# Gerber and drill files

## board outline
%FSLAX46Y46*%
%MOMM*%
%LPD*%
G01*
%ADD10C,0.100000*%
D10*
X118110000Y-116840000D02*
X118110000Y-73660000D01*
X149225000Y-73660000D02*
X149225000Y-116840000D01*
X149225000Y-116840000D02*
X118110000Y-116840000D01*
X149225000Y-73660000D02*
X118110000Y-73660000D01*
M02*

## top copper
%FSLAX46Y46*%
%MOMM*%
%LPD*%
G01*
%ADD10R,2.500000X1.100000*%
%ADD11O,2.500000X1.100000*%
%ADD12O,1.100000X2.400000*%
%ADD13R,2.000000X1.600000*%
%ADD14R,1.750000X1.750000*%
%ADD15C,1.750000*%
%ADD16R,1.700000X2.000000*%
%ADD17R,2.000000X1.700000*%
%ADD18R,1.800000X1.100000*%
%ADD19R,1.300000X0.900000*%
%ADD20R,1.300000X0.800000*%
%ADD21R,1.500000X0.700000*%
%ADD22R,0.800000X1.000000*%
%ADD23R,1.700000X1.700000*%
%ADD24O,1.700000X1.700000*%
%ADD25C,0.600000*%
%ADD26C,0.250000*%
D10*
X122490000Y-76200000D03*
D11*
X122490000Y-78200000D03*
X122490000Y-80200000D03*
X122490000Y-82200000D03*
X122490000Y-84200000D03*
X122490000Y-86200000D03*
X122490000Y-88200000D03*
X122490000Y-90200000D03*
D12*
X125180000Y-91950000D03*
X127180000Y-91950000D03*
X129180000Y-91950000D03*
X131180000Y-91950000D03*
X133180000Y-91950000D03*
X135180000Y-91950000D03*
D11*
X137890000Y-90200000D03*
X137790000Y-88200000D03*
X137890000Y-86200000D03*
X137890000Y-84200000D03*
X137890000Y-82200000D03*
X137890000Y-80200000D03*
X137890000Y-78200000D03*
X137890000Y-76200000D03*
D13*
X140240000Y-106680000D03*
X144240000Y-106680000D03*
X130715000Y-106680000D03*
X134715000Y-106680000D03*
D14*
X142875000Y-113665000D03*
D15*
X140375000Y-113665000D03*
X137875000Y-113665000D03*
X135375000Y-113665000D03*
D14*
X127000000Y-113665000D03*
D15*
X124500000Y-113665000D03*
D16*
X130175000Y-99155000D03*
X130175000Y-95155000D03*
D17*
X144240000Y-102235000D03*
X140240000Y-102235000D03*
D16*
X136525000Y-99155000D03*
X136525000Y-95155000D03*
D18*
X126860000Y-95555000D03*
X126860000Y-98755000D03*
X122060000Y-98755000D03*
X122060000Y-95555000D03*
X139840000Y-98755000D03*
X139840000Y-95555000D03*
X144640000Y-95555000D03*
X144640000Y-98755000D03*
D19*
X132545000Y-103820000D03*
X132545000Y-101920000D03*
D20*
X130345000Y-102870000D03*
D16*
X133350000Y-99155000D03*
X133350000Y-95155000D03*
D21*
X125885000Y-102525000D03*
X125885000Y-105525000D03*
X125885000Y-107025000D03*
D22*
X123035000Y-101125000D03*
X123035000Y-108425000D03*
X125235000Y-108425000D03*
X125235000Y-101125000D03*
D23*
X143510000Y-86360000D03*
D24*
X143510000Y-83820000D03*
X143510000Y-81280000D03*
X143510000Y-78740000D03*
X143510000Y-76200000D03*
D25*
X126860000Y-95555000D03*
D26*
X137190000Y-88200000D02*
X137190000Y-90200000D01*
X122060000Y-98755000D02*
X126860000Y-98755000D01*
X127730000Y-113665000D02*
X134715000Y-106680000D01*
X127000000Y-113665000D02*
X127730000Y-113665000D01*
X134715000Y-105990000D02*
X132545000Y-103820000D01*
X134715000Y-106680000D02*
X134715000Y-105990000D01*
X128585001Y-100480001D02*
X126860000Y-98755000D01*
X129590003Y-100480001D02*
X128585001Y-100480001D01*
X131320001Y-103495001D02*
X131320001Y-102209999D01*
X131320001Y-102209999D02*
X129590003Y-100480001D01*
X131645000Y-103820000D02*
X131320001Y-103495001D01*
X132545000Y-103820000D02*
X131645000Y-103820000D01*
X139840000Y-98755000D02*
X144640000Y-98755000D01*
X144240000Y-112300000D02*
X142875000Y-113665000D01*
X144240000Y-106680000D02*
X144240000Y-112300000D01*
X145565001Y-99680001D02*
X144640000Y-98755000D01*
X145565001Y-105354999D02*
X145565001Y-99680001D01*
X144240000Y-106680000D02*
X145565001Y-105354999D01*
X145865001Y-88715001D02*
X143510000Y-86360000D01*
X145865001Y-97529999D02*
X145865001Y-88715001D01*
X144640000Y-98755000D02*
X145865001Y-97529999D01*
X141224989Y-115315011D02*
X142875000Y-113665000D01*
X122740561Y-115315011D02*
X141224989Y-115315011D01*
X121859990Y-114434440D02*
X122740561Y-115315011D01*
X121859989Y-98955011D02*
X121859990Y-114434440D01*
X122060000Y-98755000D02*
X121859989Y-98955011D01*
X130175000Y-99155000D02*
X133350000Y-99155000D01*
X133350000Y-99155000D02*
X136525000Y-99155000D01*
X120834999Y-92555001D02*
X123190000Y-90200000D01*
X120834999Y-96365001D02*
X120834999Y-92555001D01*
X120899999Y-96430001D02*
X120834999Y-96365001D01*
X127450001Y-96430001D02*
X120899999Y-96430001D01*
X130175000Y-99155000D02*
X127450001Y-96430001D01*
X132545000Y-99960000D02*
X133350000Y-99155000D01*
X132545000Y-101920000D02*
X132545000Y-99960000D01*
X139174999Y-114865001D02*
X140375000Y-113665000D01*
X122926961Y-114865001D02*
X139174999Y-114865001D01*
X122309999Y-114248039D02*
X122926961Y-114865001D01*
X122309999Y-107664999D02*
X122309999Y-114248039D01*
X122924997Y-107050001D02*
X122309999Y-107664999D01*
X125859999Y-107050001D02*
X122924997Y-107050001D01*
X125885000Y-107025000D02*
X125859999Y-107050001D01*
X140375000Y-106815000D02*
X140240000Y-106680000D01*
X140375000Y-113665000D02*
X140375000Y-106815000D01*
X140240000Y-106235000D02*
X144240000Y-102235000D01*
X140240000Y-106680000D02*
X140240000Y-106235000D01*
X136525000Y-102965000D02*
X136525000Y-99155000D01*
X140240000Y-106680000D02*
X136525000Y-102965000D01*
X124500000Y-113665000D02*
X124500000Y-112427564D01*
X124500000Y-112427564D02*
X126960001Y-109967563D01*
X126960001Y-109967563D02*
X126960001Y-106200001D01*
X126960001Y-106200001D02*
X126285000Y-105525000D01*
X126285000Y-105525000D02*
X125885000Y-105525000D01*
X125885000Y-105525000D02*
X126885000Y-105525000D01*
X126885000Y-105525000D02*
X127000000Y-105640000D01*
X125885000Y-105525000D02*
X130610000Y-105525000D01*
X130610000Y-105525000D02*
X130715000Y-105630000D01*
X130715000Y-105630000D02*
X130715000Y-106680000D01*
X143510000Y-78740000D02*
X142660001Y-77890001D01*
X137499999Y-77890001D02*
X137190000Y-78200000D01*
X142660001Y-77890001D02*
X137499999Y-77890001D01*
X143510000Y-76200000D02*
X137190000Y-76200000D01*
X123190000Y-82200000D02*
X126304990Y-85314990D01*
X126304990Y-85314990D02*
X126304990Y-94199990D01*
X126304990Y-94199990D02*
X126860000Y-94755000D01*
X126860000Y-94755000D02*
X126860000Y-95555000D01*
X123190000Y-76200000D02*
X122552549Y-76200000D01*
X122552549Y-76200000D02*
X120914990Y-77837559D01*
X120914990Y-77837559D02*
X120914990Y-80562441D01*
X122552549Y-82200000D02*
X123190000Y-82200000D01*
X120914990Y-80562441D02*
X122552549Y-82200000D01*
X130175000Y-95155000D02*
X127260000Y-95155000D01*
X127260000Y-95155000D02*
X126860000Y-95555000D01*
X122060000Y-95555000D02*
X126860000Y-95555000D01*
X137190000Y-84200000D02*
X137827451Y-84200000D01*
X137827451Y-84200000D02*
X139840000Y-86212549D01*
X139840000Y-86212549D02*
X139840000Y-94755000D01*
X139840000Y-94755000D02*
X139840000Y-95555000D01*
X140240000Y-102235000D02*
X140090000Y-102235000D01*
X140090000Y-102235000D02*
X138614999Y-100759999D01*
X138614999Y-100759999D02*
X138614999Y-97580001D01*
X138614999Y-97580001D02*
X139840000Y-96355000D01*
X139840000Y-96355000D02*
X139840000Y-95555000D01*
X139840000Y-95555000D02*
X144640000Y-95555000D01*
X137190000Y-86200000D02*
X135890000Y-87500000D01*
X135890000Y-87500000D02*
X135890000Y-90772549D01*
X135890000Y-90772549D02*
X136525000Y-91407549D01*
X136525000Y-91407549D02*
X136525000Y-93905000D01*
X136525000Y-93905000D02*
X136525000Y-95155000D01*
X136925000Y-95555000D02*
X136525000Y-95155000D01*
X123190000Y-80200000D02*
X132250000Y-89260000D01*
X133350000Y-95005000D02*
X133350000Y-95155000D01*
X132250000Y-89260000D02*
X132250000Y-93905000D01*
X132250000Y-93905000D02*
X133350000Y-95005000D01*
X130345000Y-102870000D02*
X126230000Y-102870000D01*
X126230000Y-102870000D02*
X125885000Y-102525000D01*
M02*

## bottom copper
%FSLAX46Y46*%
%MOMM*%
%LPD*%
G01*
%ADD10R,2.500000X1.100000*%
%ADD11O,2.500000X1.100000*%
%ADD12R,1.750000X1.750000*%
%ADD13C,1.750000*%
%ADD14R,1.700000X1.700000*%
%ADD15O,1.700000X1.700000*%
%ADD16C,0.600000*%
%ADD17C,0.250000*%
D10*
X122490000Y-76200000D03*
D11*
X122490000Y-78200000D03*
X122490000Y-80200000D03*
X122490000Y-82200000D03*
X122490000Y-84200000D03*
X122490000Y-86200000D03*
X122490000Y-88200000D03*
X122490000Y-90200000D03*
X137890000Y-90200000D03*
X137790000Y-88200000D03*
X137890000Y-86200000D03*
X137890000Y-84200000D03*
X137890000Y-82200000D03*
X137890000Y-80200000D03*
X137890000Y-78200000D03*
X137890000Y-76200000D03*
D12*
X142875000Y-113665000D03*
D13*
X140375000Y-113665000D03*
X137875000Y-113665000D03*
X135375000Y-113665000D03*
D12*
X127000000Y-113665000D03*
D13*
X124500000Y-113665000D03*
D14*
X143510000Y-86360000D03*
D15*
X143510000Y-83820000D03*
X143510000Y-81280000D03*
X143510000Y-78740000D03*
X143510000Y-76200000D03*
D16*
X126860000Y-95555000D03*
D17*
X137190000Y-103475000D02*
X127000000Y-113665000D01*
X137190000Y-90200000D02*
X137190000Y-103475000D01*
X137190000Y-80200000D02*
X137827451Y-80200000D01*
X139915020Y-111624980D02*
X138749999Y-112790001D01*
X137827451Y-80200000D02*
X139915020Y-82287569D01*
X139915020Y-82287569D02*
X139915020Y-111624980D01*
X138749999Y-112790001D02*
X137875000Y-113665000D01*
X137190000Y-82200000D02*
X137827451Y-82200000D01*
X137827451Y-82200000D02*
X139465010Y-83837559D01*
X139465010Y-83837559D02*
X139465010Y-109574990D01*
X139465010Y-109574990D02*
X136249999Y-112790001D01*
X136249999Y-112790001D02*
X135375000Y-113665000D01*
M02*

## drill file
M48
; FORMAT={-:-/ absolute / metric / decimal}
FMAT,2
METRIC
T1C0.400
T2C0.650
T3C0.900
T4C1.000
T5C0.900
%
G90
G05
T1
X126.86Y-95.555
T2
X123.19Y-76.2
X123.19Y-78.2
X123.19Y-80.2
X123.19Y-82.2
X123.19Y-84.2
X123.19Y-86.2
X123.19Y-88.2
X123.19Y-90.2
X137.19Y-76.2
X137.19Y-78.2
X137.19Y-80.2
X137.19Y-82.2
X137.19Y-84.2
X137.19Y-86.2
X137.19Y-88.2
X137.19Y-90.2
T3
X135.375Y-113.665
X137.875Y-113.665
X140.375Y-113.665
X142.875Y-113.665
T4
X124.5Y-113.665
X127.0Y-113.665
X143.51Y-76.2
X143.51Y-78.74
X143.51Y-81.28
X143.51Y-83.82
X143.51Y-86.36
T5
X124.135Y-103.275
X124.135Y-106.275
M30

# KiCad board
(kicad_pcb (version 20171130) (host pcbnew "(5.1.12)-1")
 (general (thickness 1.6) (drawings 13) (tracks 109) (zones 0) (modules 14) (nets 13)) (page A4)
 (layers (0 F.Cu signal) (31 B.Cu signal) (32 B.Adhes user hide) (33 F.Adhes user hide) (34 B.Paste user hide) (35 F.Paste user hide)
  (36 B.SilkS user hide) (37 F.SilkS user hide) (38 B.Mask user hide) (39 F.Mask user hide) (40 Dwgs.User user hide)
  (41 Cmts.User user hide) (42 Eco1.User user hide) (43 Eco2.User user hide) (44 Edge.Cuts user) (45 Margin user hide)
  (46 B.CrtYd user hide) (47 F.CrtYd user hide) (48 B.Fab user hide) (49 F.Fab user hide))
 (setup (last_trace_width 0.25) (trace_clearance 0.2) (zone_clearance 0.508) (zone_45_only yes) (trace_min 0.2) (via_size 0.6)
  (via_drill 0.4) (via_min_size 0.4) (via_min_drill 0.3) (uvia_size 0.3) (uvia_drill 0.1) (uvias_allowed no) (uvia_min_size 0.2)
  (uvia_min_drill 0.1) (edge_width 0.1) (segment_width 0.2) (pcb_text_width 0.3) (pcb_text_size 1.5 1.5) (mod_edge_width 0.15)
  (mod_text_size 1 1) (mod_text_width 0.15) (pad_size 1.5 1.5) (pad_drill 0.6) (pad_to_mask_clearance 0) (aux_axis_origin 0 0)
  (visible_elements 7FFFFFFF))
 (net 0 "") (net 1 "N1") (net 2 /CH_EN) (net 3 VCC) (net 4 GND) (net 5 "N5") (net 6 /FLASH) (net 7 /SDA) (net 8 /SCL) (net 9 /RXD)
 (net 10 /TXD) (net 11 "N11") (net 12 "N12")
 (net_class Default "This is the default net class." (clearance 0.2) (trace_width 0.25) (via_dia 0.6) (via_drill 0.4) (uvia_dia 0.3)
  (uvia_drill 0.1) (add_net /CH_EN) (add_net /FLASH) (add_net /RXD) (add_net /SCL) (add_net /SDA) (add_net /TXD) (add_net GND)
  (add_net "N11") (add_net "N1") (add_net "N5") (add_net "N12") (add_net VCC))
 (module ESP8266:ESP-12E (layer F.Cu) (at 123.19 76.2)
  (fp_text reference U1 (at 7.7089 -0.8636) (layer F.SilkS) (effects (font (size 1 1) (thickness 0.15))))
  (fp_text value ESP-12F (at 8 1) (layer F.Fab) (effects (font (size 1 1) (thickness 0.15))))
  (pad 1 thru_hole rect (at 0 0) (size 2.5 1.1) (drill 0.65 (offset -0.7 0)) (layers *.Cu *.Mask F.SilkS) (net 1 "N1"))
  (pad 2 thru_hole oval (at 0 2) (size 2.5 1.1) (drill 0.65 (offset -0.7 0)) (layers *.Cu *.Mask F.SilkS))
  (pad 3 thru_hole oval (at 0 4) (size 2.5 1.1) (drill 0.65 (offset -0.7 0)) (layers *.Cu *.Mask F.SilkS) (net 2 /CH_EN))
  (pad 4 thru_hole oval (at 0 6) (size 2.5 1.1) (drill 0.65 (offset -0.7 0)) (layers *.Cu *.Mask F.SilkS) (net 1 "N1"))
  (pad 5 thru_hole oval (at 0 8) (size 2.5 1.1) (drill 0.65 (offset -0.7 0)) (layers *.Cu *.Mask F.SilkS))
  (pad 6 thru_hole oval (at 0 10) (size 2.5 1.1) (drill 0.65 (offset -0.7 0)) (layers *.Cu *.Mask F.SilkS))
  (pad 7 thru_hole oval (at 0 12) (size 2.5 1.1) (drill 0.65 (offset -0.7 0)) (layers *.Cu *.Mask F.SilkS))
  (pad 8 thru_hole oval (at 0 14) (size 2.5 1.1) (drill 0.65 (offset -0.7 0)) (layers *.Cu *.Mask F.SilkS) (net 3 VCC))
  (pad 9 smd oval (at 1.99 15.75 90) (size 2.4 1.1) (layers F.Cu F.Paste F.Mask))
  (pad 10 smd oval (at 3.99 15.75 90) (size 2.4 1.1) (layers F.Cu F.Paste F.Mask))
  (pad 11 smd oval (at 5.99 15.75 90) (size 2.4 1.1) (layers F.Cu F.Paste F.Mask))
  (pad 12 smd oval (at 7.99 15.75 90) (size 2.4 1.1) (layers F.Cu F.Paste F.Mask))
  (pad 13 smd oval (at 9.99 15.75 90) (size 2.4 1.1) (layers F.Cu F.Paste F.Mask))
  (pad 14 smd oval (at 11.99 15.75 90) (size 2.4 1.1) (layers F.Cu F.Paste F.Mask))
  (pad 15 thru_hole oval (at 14 14) (size 2.5 1.1) (drill 0.65 (offset 0.7 0)) (layers *.Cu *.Mask F.SilkS) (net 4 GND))
  (pad 16 thru_hole oval (at 14 12) (size 2.5 1.1) (drill 0.65 (offset 0.6 0)) (layers *.Cu *.Mask F.SilkS) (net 4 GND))
  (pad 17 thru_hole oval (at 14 10) (size 2.5 1.1) (drill 0.65 (offset 0.7 0)) (layers *.Cu *.Mask F.SilkS) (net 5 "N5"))
  (pad 18 thru_hole oval (at 14 8) (size 2.5 1.1) (drill 0.65 (offset 0.7 0)) (layers *.Cu *.Mask F.SilkS) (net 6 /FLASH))
  (pad 19 thru_hole oval (at 14 6) (size 2.5 1.1) (drill 0.65 (offset 0.7 0)) (layers *.Cu *.Mask F.SilkS) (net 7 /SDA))
  (pad 20 thru_hole oval (at 14 4) (size 2.5 1.1) (drill 0.65 (offset 0.7 0)) (layers *.Cu *.Mask F.SilkS) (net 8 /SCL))
  (pad 21 thru_hole oval (at 14 2) (size 2.5 1.1) (drill 0.65 (offset 0.7 0)) (layers *.Cu *.Mask F.SilkS) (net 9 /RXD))
  (pad 22 thru_hole oval (at 14 0) (size 2.5 1.1) (drill 0.65 (offset 0.7 0)) (layers *.Cu *.Mask F.SilkS) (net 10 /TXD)))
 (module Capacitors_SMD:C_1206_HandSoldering (layer F.Cu) (at 142.24 106.68)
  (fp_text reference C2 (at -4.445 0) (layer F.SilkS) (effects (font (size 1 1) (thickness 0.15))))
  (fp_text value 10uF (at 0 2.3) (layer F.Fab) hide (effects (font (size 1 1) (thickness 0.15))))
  (pad 1 smd rect (at -2 0) (size 2 1.6) (layers F.Cu F.Paste F.Mask) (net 3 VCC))
  (pad 2 smd rect (at 2 0) (size 2 1.6) (layers F.Cu F.Paste F.Mask) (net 4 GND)))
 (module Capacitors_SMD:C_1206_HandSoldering (layer F.Cu) (at 132.715 106.68)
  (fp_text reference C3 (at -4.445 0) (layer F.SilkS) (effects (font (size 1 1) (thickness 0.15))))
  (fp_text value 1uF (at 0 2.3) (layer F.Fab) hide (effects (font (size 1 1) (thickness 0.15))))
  (pad 1 smd rect (at -2 0) (size 2 1.6) (layers F.Cu F.Paste F.Mask) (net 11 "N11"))
  (pad 2 smd rect (at 2 0) (size 2 1.6) (layers F.Cu F.Paste F.Mask) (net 4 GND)))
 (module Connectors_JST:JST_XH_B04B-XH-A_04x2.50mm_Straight (layer F.Cu) (at 142.875 113.665 180)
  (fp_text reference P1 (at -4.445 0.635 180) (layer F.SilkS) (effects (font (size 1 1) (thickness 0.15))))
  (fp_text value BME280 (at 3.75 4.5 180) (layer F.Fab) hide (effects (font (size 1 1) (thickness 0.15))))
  (pad 1 thru_hole rect (at 0 0 180) (size 1.75 1.75) (drill 0.9) (layers *.Cu *.Mask) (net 4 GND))
  (pad 2 thru_hole circle (at 2.5 0 180) (size 1.75 1.75) (drill 0.9) (layers *.Cu *.Mask) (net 3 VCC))
  (pad 3 thru_hole circle (at 5 0 180) (size 1.75 1.75) (drill 0.9) (layers *.Cu *.Mask) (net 8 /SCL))
  (pad 4 thru_hole circle (at 7.5 0 180) (size 1.75 1.75) (drill 0.9) (layers *.Cu *.Mask) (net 7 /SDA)))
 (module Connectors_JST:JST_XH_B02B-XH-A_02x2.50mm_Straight (layer F.Cu) (at 127 113.665 180)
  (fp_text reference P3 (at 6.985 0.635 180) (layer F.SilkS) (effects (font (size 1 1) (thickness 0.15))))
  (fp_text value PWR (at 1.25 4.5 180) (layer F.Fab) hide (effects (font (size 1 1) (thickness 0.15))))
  (pad 1 thru_hole rect (at 0 0 180) (size 1.75 1.75) (drill 1) (layers *.Cu *.Mask) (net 4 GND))
  (pad 2 thru_hole circle (at 2.5 0 180) (size 1.75 1.75) (drill 1) (layers *.Cu *.Mask) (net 11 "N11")))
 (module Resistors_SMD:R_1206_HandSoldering (layer F.Cu) (at 130.175 97.155 90)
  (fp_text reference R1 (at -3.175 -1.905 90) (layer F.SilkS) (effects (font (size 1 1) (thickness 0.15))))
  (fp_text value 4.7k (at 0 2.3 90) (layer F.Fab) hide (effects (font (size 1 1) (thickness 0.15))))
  (pad 1 smd rect (at -2 0 90) (size 2 1.7) (layers F.Cu F.Paste F.Mask) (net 3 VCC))
  (pad 2 smd rect (at 2 0 90) (size 2 1.7) (layers F.Cu F.Paste F.Mask) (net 1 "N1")))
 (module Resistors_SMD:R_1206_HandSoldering (layer F.Cu) (at 142.24 102.235 180)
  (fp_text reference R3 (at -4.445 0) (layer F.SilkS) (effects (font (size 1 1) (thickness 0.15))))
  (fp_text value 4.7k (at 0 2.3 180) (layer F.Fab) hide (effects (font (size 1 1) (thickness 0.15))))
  (pad 1 smd rect (at -2 0 180) (size 2 1.7) (layers F.Cu F.Paste F.Mask) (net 3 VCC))
  (pad 2 smd rect (at 2 0 180) (size 2 1.7) (layers F.Cu F.Paste F.Mask) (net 6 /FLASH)))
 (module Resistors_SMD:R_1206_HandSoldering (layer F.Cu) (at 136.525 97.155 90)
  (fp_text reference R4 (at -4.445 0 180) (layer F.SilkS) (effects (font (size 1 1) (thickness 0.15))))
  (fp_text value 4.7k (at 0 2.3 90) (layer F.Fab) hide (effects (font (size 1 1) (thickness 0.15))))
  (pad 1 smd rect (at -2 0 90) (size 2 1.7) (layers F.Cu F.Paste F.Mask) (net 3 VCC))
  (pad 2 smd rect (at 2 0 90) (size 2 1.7) (layers F.Cu F.Paste F.Mask) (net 5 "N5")))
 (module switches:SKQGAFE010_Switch (layer F.Cu) (at 124.46 97.155 180)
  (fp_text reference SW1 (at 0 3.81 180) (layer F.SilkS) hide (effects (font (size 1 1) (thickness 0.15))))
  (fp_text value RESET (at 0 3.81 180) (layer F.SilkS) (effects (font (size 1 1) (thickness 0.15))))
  (pad 3 smd rect (at -2.4 1.6 180) (size 1.8 1.1) (layers F.Cu F.Paste F.Mask) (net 1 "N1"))
  (pad 1 smd rect (at -2.4 -1.6 180) (size 1.8 1.1) (layers F.Cu F.Paste F.Mask) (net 4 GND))
  (pad 2 smd rect (at 2.4 -1.6 180) (size 1.8 1.1) (layers F.Cu F.Paste F.Mask) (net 4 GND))
  (pad 4 smd rect (at 2.4 1.6 180) (size 1.8 1.1) (layers F.Cu F.Paste F.Mask) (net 1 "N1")))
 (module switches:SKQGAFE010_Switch (layer F.Cu) (at 142.24 97.155)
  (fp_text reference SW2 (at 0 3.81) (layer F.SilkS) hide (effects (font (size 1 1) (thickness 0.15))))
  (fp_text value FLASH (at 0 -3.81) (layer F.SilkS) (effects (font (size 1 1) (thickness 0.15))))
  (pad 3 smd rect (at -2.4 1.6) (size 1.8 1.1) (layers F.Cu F.Paste F.Mask) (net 4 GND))
  (pad 1 smd rect (at -2.4 -1.6) (size 1.8 1.1) (layers F.Cu F.Paste F.Mask) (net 6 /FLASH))
  (pad 2 smd rect (at 2.4 -1.6) (size 1.8 1.1) (layers F.Cu F.Paste F.Mask) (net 6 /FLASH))
  (pad 4 smd rect (at 2.4 1.6) (size 1.8 1.1) (layers F.Cu F.Paste F.Mask) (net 4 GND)))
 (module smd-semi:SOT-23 (layer F.Cu) (at 131.445 102.87 180)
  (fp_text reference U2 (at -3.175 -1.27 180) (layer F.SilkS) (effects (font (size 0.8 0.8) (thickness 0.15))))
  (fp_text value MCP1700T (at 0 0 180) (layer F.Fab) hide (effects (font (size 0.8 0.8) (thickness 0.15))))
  (pad 1 smd rect (at -1.1 -0.95 180) (size 1.3 0.9) (layers F.Cu F.Paste F.Mask) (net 4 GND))
  (pad 2 smd rect (at -1.1 0.95 180) (size 1.3 0.9) (layers F.Cu F.Paste F.Mask) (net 3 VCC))
  (pad 3 smd rect (at 1.1 0 180) (size 1.3 0.8) (layers F.Cu F.Paste F.Mask) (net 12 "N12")))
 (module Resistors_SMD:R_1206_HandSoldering (layer F.Cu) (at 133.35 97.155 90)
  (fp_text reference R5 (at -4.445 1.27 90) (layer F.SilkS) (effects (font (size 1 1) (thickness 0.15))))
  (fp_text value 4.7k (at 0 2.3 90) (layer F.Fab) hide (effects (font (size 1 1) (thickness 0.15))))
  (pad 1 smd rect (at -2 0 90) (size 2 1.7) (layers F.Cu F.Paste F.Mask) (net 3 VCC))
  (pad 2 smd rect (at 2 0 90) (size 2 1.7) (layers F.Cu F.Paste F.Mask) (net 2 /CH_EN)))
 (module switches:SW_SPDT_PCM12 (layer F.Cu) (at 124.46 104.775 270)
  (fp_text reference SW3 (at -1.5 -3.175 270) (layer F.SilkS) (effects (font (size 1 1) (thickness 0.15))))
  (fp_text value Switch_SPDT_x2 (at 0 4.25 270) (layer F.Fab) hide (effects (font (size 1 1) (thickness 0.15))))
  (pad "" np_thru_hole circle (at -1.5 0.325 270) (size 0.9 0.9) (drill 0.9) (layers *.Cu *.Mask))
  (pad "" np_thru_hole circle (at 1.5 0.325 270) (size 0.9 0.9) (drill 0.9) (layers *.Cu *.Mask))
  (pad 1 smd rect (at -2.25 -1.425 270) (size 0.7 1.5) (layers F.Cu F.Paste F.Mask) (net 12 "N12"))
  (pad 2 smd rect (at 0.75 -1.425 270) (size 0.7 1.5) (layers F.Cu F.Paste F.Mask) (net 11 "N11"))
  (pad 3 smd rect (at 2.25 -1.425 270) (size 0.7 1.5) (layers F.Cu F.Paste F.Mask) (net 3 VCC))
  (pad "" smd rect (at -3.65 1.425 270) (size 1 0.8) (layers F.Cu F.Paste F.Mask))
  (pad "" smd rect (at 3.65 1.425 270) (size 1 0.8) (layers F.Cu F.Paste F.Mask))
  (pad "" smd rect (at 3.65 -0.775 270) (size 1 0.8) (layers F.Cu F.Paste F.Mask))
  (pad "" smd rect (at -3.65 -0.775 270) (size 1 0.8) (layers F.Cu F.Paste F.Mask)))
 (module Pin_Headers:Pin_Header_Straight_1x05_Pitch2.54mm (layer F.Cu) (at 143.51 86.36 180)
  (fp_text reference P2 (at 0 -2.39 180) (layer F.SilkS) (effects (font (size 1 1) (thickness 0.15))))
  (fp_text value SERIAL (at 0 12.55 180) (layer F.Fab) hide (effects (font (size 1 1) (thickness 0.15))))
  (pad 1 thru_hole rect (at 0 0 180) (size 1.7 1.7) (drill 1) (layers *.Cu *.Mask) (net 4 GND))
  (pad 2 thru_hole oval (at 0 2.54 180) (size 1.7 1.7) (drill 1) (layers *.Cu *.Mask))
  (pad 3 thru_hole oval (at 0 5.08 180) (size 1.7 1.7) (drill 1) (layers *.Cu *.Mask))
  (pad 4 thru_hole oval (at 0 7.62 180) (size 1.7 1.7) (drill 1) (layers *.Cu *.Mask) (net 9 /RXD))
  (pad 5 thru_hole oval (at 0 10.16 180) (size 1.7 1.7) (drill 1) (layers *.Cu *.Mask) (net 10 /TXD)))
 (gr_line (start 118.11 116.84) (end 118.11 73.66) (layer Edge.Cuts) (width 0.1))
 (gr_line (start 149.225 73.66) (end 149.225 116.84) (layer Edge.Cuts) (width 0.1))
 (gr_line (start 149.225 116.84) (end 118.11 116.84) (layer Edge.Cuts) (width 0.1))
 (gr_line (start 149.225 73.66) (end 118.11 73.66) (layer Edge.Cuts) (width 0.1))
 (segment (start 137.19 88.2) (end 137.19 90.2) (width 0.25) (layer F.Cu) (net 4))
 (segment (start 122.06 98.755) (end 126.86 98.755) (width 0.25) (layer F.Cu) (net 4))
 (segment (start 127.73 113.665) (end 134.715 106.68) (width 0.25) (layer F.Cu) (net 4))
 (segment (start 127 113.665) (end 127.73 113.665) (width 0.25) (layer F.Cu) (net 4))
 (segment (start 134.715 105.99) (end 132.545 103.82) (width 0.25) (layer F.Cu) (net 4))
 (segment (start 134.715 106.68) (end 134.715 105.99) (width 0.25) (layer F.Cu) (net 4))
 (segment (start 128.585001 100.480001) (end 126.86 98.755) (width 0.25) (layer F.Cu) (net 4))
 (segment (start 129.590003 100.480001) (end 128.585001 100.480001) (width 0.25) (layer F.Cu) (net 4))
 (segment (start 131.320001 103.495001) (end 131.320001 102.209999) (width 0.25) (layer F.Cu) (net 4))
 (segment (start 131.320001 102.209999) (end 129.590003 100.480001) (width 0.25) (layer F.Cu) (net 4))
 (segment (start 131.645 103.82) (end 131.320001 103.495001) (width 0.25) (layer F.Cu) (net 4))
 (segment (start 132.545 103.82) (end 131.645 103.82) (width 0.25) (layer F.Cu) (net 4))
 (segment (start 139.84 98.755) (end 144.64 98.755) (width 0.25) (layer F.Cu) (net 4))
 (segment (start 144.24 112.3) (end 142.875 113.665) (width 0.25) (layer F.Cu) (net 4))
 (segment (start 144.24 106.68) (end 144.24 112.3) (width 0.25) (layer F.Cu) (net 4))
 (segment (start 145.565001 99.680001) (end 144.64 98.755) (width 0.25) (layer F.Cu) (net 4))
 (segment (start 145.565001 105.354999) (end 145.565001 99.680001) (width 0.25) (layer F.Cu) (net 4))
 (segment (start 144.24 106.68) (end 145.565001 105.354999) (width 0.25) (layer F.Cu) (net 4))
 (segment (start 145.865001 88.715001) (end 143.51 86.36) (width 0.25) (layer F.Cu) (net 4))
 (segment (start 145.865001 97.529999) (end 145.865001 88.715001) (width 0.25) (layer F.Cu) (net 4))
 (segment (start 144.64 98.755) (end 145.865001 97.529999) (width 0.25) (layer F.Cu) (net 4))
 (segment (start 137.19 103.475) (end 127 113.665) (width 0.25) (layer B.Cu) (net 4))
 (segment (start 137.19 90.2) (end 137.19 103.475) (width 0.25) (layer B.Cu) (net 4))
 (segment (start 141.224989 115.315011) (end 142.875 113.665) (width 0.25) (layer F.Cu) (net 4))
 (segment (start 122.740561 115.315011) (end 141.224989 115.315011) (width 0.25) (layer F.Cu) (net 4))
 (segment (start 121.85999 114.43444) (end 122.740561 115.315011) (width 0.25) (layer F.Cu) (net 4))
 (segment (start 121.859989 98.955011) (end 121.85999 114.43444) (width 0.25) (layer F.Cu) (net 4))
 (segment (start 122.06 98.755) (end 121.859989 98.955011) (width 0.25) (layer F.Cu) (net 4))
 (segment (start 130.175 99.155) (end 133.35 99.155) (width 0.25) (layer F.Cu) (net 3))
 (segment (start 133.35 99.155) (end 136.525 99.155) (width 0.25) (layer F.Cu) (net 3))
 (segment (start 120.834999 92.555001) (end 123.19 90.2) (width 0.25) (layer F.Cu) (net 3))
 (segment (start 120.834999 96.365001) (end 120.834999 92.555001) (width 0.25) (layer F.Cu) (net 3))
 (segment (start 120.899999 96.430001) (end 120.834999 96.365001) (width 0.25) (layer F.Cu) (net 3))
 (segment (start 127.450001 96.430001) (end 120.899999 96.430001) (width 0.25) (layer F.Cu) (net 3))
 (segment (start 130.175 99.155) (end 127.450001 96.430001) (width 0.25) (layer F.Cu) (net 3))
 (segment (start 132.545 99.96) (end 133.35 99.155) (width 0.25) (layer F.Cu) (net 3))
 (segment (start 132.545 101.92) (end 132.545 99.96) (width 0.25) (layer F.Cu) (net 3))
 (segment (start 139.174999 114.865001) (end 140.375 113.665) (width 0.25) (layer F.Cu) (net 3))
 (segment (start 122.926961 114.865001) (end 139.174999 114.865001) (width 0.25) (layer F.Cu) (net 3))
 (segment (start 122.309999 114.248039) (end 122.926961 114.865001) (width 0.25) (layer F.Cu) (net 3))
 (segment (start 122.309999 107.664999) (end 122.309999 114.248039) (width 0.25) (layer F.Cu) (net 3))
 (segment (start 122.924997 107.050001) (end 122.309999 107.664999) (width 0.25) (layer F.Cu) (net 3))
 (segment (start 125.859999 107.050001) (end 122.924997 107.050001) (width 0.25) (layer F.Cu) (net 3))
 (segment (start 125.885 107.025) (end 125.859999 107.050001) (width 0.25) (layer F.Cu) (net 3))
 (segment (start 140.375 106.815) (end 140.24 106.68) (width 0.25) (layer F.Cu) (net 3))
 (segment (start 140.375 113.665) (end 140.375 106.815) (width 0.25) (layer F.Cu) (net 3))
 (segment (start 140.24 106.235) (end 144.24 102.235) (width 0.25) (layer F.Cu) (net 3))
 (segment (start 140.24 106.68) (end 140.24 106.235) (width 0.25) (layer F.Cu) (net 3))
 (segment (start 136.525 102.965) (end 136.525 99.155) (width 0.25) (layer F.Cu) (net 3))
 (segment (start 140.24 106.68) (end 136.525 102.965) (width 0.25) (layer F.Cu) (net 3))
 (segment (start 124.5 113.665) (end 124.5 112.427564) (width 0.25) (layer F.Cu) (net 11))
 (segment (start 124.5 112.427564) (end 126.960001 109.967563) (width 0.25) (layer F.Cu) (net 11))
 (segment (start 126.960001 109.967563) (end 126.960001 106.200001) (width 0.25) (layer F.Cu) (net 11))
 (segment (start 126.960001 106.200001) (end 126.285 105.525) (width 0.25) (layer F.Cu) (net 11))
 (segment (start 126.285 105.525) (end 125.885 105.525) (width 0.25) (layer F.Cu) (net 11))
 (segment (start 125.885 105.525) (end 126.885 105.525) (width 0.25) (layer F.Cu) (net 11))
 (segment (start 126.885 105.525) (end 127 105.64) (width 0.25) (layer F.Cu) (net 11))
 (segment (start 125.885 105.525) (end 130.61 105.525) (width 0.25) (layer F.Cu) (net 11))
 (segment (start 130.61 105.525) (end 130.715 105.63) (width 0.25) (layer F.Cu) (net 11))
 (segment (start 130.715 105.63) (end 130.715 106.68) (width 0.25) (layer F.Cu) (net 11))
 (segment (start 137.19 80.2) (end 137.827451 80.2) (width 0.25) (layer B.Cu) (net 8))
 (segment (start 139.91502 111.62498) (end 138.749999 112.790001) (width 0.25) (layer B.Cu) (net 8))
 (segment (start 137.827451 80.2) (end 139.91502 82.287569) (width 0.25) (layer B.Cu) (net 8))
 (segment (start 139.91502 82.287569) (end 139.91502 111.62498) (width 0.25) (layer B.Cu) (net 8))
 (segment (start 138.749999 112.790001) (end 137.875 113.665) (width 0.25) (layer B.Cu) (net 8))
 (segment (start 137.19 82.2) (end 137.827451 82.2) (width 0.25) (layer B.Cu) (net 7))
 (segment (start 137.827451 82.2) (end 139.46501 83.837559) (width 0.25) (layer B.Cu) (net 7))
 (segment (start 139.46501 83.837559) (end 139.46501 109.57499) (width 0.25) (layer B.Cu) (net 7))
 (segment (start 139.46501 109.57499) (end 136.249999 112.790001) (width 0.25) (layer B.Cu) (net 7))
 (segment (start 136.249999 112.790001) (end 135.375 113.665) (width 0.25) (layer B.Cu) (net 7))
 (segment (start 143.51 78.74) (end 142.660001 77.890001) (width 0.25) (layer F.Cu) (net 9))
 (segment (start 137.499999 77.890001) (end 137.19 78.2) (width 0.25) (layer F.Cu) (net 9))
 (segment (start 142.660001 77.890001) (end 137.499999 77.890001) (width 0.25) (layer F.Cu) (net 9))
 (segment (start 143.51 76.2) (end 137.19 76.2) (width 0.25) (layer F.Cu) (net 10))
 (via (at 126.86 95.555) (size 0.6) (drill 0.4) (layers F.Cu B.Cu) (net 1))
 (segment (start 123.19 82.2) (end 126.30499 85.31499) (width 0.25) (layer F.Cu) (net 1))
 (segment (start 126.30499 85.31499) (end 126.30499 94.19999) (width 0.25) (layer F.Cu) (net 1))
 (segment (start 126.30499 94.19999) (end 126.86 94.755) (width 0.25) (layer F.Cu) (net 1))
 (segment (start 126.86 94.755) (end 126.86 95.555) (width 0.25) (layer F.Cu) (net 1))
 (segment (start 123.19 76.2) (end 122.552549 76.2) (width 0.25) (layer F.Cu) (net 1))
 (segment (start 122.552549 76.2) (end 120.91499 77.837559) (width 0.25) (layer F.Cu) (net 1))
 (segment (start 120.91499 77.837559) (end 120.91499 80.562441) (width 0.25) (layer F.Cu) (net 1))
 (segment (start 122.552549 82.2) (end 123.19 82.2) (width 0.25) (layer F.Cu) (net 1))
 (segment (start 120.91499 80.562441) (end 122.552549 82.2) (width 0.25) (layer F.Cu) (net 1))
 (segment (start 130.175 95.155) (end 127.26 95.155) (width 0.25) (layer F.Cu) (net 1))
 (segment (start 127.26 95.155) (end 126.86 95.555) (width 0.25) (layer F.Cu) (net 1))
 (segment (start 122.06 95.555) (end 126.86 95.555) (width 0.25) (layer F.Cu) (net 1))
 (segment (start 137.19 84.2) (end 137.827451 84.2) (width 0.25) (layer F.Cu) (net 6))
 (segment (start 137.827451 84.2) (end 139.84 86.212549) (width 0.25) (layer F.Cu) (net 6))
 (segment (start 139.84 86.212549) (end 139.84 94.755) (width 0.25) (layer F.Cu) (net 6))
 (segment (start 139.84 94.755) (end 139.84 95.555) (width 0.25) (layer F.Cu) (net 6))
 (segment (start 140.24 102.235) (end 140.09 102.235) (width 0.25) (layer F.Cu) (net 6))
 (segment (start 140.09 102.235) (end 138.614999 100.759999) (width 0.25) (layer F.Cu) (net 6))
 (segment (start 138.614999 100.759999) (end 138.614999 97.580001) (width 0.25) (layer F.Cu) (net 6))
 (segment (start 138.614999 97.580001) (end 139.84 96.355) (width 0.25) (layer F.Cu) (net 6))
 (segment (start 139.84 96.355) (end 139.84 95.555) (width 0.25) (layer F.Cu) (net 6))
 (segment (start 139.84 95.555) (end 144.64 95.555) (width 0.25) (layer F.Cu) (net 6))
 (segment (start 137.19 86.2) (end 135.89 87.5) (width 0.25) (layer F.Cu) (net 5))
 (segment (start 135.89 87.5) (end 135.89 90.772549) (width 0.25) (layer F.Cu) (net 5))
 (segment (start 135.89 90.772549) (end 136.525 91.407549) (width 0.25) (layer F.Cu) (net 5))
 (segment (start 136.525 91.407549) (end 136.525 93.905) (width 0.25) (layer F.Cu) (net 5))
 (segment (start 136.525 93.905) (end 136.525 95.155) (width 0.25) (layer F.Cu) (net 5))
 (segment (start 136.925 95.555) (end 136.525 95.155) (width 0.25) (layer F.Cu) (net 5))
 (segment (start 123.19 80.2) (end 132.25 89.26) (width 0.25) (layer F.Cu) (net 2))
 (segment (start 133.35 95.005) (end 133.35 95.155) (width 0.25) (layer F.Cu) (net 2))
 (segment (start 132.25 89.26) (end 132.25 93.905) (width 0.25) (layer F.Cu) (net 2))
 (segment (start 132.25 93.905) (end 133.35 95.005) (width 0.25) (layer F.Cu) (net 2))
 (segment (start 130.345 102.87) (end 126.23 102.87) (width 0.25) (layer F.Cu) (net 12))
 (segment (start 126.23 102.87) (end 125.885 102.525) (width 0.25) (layer F.Cu) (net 12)))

